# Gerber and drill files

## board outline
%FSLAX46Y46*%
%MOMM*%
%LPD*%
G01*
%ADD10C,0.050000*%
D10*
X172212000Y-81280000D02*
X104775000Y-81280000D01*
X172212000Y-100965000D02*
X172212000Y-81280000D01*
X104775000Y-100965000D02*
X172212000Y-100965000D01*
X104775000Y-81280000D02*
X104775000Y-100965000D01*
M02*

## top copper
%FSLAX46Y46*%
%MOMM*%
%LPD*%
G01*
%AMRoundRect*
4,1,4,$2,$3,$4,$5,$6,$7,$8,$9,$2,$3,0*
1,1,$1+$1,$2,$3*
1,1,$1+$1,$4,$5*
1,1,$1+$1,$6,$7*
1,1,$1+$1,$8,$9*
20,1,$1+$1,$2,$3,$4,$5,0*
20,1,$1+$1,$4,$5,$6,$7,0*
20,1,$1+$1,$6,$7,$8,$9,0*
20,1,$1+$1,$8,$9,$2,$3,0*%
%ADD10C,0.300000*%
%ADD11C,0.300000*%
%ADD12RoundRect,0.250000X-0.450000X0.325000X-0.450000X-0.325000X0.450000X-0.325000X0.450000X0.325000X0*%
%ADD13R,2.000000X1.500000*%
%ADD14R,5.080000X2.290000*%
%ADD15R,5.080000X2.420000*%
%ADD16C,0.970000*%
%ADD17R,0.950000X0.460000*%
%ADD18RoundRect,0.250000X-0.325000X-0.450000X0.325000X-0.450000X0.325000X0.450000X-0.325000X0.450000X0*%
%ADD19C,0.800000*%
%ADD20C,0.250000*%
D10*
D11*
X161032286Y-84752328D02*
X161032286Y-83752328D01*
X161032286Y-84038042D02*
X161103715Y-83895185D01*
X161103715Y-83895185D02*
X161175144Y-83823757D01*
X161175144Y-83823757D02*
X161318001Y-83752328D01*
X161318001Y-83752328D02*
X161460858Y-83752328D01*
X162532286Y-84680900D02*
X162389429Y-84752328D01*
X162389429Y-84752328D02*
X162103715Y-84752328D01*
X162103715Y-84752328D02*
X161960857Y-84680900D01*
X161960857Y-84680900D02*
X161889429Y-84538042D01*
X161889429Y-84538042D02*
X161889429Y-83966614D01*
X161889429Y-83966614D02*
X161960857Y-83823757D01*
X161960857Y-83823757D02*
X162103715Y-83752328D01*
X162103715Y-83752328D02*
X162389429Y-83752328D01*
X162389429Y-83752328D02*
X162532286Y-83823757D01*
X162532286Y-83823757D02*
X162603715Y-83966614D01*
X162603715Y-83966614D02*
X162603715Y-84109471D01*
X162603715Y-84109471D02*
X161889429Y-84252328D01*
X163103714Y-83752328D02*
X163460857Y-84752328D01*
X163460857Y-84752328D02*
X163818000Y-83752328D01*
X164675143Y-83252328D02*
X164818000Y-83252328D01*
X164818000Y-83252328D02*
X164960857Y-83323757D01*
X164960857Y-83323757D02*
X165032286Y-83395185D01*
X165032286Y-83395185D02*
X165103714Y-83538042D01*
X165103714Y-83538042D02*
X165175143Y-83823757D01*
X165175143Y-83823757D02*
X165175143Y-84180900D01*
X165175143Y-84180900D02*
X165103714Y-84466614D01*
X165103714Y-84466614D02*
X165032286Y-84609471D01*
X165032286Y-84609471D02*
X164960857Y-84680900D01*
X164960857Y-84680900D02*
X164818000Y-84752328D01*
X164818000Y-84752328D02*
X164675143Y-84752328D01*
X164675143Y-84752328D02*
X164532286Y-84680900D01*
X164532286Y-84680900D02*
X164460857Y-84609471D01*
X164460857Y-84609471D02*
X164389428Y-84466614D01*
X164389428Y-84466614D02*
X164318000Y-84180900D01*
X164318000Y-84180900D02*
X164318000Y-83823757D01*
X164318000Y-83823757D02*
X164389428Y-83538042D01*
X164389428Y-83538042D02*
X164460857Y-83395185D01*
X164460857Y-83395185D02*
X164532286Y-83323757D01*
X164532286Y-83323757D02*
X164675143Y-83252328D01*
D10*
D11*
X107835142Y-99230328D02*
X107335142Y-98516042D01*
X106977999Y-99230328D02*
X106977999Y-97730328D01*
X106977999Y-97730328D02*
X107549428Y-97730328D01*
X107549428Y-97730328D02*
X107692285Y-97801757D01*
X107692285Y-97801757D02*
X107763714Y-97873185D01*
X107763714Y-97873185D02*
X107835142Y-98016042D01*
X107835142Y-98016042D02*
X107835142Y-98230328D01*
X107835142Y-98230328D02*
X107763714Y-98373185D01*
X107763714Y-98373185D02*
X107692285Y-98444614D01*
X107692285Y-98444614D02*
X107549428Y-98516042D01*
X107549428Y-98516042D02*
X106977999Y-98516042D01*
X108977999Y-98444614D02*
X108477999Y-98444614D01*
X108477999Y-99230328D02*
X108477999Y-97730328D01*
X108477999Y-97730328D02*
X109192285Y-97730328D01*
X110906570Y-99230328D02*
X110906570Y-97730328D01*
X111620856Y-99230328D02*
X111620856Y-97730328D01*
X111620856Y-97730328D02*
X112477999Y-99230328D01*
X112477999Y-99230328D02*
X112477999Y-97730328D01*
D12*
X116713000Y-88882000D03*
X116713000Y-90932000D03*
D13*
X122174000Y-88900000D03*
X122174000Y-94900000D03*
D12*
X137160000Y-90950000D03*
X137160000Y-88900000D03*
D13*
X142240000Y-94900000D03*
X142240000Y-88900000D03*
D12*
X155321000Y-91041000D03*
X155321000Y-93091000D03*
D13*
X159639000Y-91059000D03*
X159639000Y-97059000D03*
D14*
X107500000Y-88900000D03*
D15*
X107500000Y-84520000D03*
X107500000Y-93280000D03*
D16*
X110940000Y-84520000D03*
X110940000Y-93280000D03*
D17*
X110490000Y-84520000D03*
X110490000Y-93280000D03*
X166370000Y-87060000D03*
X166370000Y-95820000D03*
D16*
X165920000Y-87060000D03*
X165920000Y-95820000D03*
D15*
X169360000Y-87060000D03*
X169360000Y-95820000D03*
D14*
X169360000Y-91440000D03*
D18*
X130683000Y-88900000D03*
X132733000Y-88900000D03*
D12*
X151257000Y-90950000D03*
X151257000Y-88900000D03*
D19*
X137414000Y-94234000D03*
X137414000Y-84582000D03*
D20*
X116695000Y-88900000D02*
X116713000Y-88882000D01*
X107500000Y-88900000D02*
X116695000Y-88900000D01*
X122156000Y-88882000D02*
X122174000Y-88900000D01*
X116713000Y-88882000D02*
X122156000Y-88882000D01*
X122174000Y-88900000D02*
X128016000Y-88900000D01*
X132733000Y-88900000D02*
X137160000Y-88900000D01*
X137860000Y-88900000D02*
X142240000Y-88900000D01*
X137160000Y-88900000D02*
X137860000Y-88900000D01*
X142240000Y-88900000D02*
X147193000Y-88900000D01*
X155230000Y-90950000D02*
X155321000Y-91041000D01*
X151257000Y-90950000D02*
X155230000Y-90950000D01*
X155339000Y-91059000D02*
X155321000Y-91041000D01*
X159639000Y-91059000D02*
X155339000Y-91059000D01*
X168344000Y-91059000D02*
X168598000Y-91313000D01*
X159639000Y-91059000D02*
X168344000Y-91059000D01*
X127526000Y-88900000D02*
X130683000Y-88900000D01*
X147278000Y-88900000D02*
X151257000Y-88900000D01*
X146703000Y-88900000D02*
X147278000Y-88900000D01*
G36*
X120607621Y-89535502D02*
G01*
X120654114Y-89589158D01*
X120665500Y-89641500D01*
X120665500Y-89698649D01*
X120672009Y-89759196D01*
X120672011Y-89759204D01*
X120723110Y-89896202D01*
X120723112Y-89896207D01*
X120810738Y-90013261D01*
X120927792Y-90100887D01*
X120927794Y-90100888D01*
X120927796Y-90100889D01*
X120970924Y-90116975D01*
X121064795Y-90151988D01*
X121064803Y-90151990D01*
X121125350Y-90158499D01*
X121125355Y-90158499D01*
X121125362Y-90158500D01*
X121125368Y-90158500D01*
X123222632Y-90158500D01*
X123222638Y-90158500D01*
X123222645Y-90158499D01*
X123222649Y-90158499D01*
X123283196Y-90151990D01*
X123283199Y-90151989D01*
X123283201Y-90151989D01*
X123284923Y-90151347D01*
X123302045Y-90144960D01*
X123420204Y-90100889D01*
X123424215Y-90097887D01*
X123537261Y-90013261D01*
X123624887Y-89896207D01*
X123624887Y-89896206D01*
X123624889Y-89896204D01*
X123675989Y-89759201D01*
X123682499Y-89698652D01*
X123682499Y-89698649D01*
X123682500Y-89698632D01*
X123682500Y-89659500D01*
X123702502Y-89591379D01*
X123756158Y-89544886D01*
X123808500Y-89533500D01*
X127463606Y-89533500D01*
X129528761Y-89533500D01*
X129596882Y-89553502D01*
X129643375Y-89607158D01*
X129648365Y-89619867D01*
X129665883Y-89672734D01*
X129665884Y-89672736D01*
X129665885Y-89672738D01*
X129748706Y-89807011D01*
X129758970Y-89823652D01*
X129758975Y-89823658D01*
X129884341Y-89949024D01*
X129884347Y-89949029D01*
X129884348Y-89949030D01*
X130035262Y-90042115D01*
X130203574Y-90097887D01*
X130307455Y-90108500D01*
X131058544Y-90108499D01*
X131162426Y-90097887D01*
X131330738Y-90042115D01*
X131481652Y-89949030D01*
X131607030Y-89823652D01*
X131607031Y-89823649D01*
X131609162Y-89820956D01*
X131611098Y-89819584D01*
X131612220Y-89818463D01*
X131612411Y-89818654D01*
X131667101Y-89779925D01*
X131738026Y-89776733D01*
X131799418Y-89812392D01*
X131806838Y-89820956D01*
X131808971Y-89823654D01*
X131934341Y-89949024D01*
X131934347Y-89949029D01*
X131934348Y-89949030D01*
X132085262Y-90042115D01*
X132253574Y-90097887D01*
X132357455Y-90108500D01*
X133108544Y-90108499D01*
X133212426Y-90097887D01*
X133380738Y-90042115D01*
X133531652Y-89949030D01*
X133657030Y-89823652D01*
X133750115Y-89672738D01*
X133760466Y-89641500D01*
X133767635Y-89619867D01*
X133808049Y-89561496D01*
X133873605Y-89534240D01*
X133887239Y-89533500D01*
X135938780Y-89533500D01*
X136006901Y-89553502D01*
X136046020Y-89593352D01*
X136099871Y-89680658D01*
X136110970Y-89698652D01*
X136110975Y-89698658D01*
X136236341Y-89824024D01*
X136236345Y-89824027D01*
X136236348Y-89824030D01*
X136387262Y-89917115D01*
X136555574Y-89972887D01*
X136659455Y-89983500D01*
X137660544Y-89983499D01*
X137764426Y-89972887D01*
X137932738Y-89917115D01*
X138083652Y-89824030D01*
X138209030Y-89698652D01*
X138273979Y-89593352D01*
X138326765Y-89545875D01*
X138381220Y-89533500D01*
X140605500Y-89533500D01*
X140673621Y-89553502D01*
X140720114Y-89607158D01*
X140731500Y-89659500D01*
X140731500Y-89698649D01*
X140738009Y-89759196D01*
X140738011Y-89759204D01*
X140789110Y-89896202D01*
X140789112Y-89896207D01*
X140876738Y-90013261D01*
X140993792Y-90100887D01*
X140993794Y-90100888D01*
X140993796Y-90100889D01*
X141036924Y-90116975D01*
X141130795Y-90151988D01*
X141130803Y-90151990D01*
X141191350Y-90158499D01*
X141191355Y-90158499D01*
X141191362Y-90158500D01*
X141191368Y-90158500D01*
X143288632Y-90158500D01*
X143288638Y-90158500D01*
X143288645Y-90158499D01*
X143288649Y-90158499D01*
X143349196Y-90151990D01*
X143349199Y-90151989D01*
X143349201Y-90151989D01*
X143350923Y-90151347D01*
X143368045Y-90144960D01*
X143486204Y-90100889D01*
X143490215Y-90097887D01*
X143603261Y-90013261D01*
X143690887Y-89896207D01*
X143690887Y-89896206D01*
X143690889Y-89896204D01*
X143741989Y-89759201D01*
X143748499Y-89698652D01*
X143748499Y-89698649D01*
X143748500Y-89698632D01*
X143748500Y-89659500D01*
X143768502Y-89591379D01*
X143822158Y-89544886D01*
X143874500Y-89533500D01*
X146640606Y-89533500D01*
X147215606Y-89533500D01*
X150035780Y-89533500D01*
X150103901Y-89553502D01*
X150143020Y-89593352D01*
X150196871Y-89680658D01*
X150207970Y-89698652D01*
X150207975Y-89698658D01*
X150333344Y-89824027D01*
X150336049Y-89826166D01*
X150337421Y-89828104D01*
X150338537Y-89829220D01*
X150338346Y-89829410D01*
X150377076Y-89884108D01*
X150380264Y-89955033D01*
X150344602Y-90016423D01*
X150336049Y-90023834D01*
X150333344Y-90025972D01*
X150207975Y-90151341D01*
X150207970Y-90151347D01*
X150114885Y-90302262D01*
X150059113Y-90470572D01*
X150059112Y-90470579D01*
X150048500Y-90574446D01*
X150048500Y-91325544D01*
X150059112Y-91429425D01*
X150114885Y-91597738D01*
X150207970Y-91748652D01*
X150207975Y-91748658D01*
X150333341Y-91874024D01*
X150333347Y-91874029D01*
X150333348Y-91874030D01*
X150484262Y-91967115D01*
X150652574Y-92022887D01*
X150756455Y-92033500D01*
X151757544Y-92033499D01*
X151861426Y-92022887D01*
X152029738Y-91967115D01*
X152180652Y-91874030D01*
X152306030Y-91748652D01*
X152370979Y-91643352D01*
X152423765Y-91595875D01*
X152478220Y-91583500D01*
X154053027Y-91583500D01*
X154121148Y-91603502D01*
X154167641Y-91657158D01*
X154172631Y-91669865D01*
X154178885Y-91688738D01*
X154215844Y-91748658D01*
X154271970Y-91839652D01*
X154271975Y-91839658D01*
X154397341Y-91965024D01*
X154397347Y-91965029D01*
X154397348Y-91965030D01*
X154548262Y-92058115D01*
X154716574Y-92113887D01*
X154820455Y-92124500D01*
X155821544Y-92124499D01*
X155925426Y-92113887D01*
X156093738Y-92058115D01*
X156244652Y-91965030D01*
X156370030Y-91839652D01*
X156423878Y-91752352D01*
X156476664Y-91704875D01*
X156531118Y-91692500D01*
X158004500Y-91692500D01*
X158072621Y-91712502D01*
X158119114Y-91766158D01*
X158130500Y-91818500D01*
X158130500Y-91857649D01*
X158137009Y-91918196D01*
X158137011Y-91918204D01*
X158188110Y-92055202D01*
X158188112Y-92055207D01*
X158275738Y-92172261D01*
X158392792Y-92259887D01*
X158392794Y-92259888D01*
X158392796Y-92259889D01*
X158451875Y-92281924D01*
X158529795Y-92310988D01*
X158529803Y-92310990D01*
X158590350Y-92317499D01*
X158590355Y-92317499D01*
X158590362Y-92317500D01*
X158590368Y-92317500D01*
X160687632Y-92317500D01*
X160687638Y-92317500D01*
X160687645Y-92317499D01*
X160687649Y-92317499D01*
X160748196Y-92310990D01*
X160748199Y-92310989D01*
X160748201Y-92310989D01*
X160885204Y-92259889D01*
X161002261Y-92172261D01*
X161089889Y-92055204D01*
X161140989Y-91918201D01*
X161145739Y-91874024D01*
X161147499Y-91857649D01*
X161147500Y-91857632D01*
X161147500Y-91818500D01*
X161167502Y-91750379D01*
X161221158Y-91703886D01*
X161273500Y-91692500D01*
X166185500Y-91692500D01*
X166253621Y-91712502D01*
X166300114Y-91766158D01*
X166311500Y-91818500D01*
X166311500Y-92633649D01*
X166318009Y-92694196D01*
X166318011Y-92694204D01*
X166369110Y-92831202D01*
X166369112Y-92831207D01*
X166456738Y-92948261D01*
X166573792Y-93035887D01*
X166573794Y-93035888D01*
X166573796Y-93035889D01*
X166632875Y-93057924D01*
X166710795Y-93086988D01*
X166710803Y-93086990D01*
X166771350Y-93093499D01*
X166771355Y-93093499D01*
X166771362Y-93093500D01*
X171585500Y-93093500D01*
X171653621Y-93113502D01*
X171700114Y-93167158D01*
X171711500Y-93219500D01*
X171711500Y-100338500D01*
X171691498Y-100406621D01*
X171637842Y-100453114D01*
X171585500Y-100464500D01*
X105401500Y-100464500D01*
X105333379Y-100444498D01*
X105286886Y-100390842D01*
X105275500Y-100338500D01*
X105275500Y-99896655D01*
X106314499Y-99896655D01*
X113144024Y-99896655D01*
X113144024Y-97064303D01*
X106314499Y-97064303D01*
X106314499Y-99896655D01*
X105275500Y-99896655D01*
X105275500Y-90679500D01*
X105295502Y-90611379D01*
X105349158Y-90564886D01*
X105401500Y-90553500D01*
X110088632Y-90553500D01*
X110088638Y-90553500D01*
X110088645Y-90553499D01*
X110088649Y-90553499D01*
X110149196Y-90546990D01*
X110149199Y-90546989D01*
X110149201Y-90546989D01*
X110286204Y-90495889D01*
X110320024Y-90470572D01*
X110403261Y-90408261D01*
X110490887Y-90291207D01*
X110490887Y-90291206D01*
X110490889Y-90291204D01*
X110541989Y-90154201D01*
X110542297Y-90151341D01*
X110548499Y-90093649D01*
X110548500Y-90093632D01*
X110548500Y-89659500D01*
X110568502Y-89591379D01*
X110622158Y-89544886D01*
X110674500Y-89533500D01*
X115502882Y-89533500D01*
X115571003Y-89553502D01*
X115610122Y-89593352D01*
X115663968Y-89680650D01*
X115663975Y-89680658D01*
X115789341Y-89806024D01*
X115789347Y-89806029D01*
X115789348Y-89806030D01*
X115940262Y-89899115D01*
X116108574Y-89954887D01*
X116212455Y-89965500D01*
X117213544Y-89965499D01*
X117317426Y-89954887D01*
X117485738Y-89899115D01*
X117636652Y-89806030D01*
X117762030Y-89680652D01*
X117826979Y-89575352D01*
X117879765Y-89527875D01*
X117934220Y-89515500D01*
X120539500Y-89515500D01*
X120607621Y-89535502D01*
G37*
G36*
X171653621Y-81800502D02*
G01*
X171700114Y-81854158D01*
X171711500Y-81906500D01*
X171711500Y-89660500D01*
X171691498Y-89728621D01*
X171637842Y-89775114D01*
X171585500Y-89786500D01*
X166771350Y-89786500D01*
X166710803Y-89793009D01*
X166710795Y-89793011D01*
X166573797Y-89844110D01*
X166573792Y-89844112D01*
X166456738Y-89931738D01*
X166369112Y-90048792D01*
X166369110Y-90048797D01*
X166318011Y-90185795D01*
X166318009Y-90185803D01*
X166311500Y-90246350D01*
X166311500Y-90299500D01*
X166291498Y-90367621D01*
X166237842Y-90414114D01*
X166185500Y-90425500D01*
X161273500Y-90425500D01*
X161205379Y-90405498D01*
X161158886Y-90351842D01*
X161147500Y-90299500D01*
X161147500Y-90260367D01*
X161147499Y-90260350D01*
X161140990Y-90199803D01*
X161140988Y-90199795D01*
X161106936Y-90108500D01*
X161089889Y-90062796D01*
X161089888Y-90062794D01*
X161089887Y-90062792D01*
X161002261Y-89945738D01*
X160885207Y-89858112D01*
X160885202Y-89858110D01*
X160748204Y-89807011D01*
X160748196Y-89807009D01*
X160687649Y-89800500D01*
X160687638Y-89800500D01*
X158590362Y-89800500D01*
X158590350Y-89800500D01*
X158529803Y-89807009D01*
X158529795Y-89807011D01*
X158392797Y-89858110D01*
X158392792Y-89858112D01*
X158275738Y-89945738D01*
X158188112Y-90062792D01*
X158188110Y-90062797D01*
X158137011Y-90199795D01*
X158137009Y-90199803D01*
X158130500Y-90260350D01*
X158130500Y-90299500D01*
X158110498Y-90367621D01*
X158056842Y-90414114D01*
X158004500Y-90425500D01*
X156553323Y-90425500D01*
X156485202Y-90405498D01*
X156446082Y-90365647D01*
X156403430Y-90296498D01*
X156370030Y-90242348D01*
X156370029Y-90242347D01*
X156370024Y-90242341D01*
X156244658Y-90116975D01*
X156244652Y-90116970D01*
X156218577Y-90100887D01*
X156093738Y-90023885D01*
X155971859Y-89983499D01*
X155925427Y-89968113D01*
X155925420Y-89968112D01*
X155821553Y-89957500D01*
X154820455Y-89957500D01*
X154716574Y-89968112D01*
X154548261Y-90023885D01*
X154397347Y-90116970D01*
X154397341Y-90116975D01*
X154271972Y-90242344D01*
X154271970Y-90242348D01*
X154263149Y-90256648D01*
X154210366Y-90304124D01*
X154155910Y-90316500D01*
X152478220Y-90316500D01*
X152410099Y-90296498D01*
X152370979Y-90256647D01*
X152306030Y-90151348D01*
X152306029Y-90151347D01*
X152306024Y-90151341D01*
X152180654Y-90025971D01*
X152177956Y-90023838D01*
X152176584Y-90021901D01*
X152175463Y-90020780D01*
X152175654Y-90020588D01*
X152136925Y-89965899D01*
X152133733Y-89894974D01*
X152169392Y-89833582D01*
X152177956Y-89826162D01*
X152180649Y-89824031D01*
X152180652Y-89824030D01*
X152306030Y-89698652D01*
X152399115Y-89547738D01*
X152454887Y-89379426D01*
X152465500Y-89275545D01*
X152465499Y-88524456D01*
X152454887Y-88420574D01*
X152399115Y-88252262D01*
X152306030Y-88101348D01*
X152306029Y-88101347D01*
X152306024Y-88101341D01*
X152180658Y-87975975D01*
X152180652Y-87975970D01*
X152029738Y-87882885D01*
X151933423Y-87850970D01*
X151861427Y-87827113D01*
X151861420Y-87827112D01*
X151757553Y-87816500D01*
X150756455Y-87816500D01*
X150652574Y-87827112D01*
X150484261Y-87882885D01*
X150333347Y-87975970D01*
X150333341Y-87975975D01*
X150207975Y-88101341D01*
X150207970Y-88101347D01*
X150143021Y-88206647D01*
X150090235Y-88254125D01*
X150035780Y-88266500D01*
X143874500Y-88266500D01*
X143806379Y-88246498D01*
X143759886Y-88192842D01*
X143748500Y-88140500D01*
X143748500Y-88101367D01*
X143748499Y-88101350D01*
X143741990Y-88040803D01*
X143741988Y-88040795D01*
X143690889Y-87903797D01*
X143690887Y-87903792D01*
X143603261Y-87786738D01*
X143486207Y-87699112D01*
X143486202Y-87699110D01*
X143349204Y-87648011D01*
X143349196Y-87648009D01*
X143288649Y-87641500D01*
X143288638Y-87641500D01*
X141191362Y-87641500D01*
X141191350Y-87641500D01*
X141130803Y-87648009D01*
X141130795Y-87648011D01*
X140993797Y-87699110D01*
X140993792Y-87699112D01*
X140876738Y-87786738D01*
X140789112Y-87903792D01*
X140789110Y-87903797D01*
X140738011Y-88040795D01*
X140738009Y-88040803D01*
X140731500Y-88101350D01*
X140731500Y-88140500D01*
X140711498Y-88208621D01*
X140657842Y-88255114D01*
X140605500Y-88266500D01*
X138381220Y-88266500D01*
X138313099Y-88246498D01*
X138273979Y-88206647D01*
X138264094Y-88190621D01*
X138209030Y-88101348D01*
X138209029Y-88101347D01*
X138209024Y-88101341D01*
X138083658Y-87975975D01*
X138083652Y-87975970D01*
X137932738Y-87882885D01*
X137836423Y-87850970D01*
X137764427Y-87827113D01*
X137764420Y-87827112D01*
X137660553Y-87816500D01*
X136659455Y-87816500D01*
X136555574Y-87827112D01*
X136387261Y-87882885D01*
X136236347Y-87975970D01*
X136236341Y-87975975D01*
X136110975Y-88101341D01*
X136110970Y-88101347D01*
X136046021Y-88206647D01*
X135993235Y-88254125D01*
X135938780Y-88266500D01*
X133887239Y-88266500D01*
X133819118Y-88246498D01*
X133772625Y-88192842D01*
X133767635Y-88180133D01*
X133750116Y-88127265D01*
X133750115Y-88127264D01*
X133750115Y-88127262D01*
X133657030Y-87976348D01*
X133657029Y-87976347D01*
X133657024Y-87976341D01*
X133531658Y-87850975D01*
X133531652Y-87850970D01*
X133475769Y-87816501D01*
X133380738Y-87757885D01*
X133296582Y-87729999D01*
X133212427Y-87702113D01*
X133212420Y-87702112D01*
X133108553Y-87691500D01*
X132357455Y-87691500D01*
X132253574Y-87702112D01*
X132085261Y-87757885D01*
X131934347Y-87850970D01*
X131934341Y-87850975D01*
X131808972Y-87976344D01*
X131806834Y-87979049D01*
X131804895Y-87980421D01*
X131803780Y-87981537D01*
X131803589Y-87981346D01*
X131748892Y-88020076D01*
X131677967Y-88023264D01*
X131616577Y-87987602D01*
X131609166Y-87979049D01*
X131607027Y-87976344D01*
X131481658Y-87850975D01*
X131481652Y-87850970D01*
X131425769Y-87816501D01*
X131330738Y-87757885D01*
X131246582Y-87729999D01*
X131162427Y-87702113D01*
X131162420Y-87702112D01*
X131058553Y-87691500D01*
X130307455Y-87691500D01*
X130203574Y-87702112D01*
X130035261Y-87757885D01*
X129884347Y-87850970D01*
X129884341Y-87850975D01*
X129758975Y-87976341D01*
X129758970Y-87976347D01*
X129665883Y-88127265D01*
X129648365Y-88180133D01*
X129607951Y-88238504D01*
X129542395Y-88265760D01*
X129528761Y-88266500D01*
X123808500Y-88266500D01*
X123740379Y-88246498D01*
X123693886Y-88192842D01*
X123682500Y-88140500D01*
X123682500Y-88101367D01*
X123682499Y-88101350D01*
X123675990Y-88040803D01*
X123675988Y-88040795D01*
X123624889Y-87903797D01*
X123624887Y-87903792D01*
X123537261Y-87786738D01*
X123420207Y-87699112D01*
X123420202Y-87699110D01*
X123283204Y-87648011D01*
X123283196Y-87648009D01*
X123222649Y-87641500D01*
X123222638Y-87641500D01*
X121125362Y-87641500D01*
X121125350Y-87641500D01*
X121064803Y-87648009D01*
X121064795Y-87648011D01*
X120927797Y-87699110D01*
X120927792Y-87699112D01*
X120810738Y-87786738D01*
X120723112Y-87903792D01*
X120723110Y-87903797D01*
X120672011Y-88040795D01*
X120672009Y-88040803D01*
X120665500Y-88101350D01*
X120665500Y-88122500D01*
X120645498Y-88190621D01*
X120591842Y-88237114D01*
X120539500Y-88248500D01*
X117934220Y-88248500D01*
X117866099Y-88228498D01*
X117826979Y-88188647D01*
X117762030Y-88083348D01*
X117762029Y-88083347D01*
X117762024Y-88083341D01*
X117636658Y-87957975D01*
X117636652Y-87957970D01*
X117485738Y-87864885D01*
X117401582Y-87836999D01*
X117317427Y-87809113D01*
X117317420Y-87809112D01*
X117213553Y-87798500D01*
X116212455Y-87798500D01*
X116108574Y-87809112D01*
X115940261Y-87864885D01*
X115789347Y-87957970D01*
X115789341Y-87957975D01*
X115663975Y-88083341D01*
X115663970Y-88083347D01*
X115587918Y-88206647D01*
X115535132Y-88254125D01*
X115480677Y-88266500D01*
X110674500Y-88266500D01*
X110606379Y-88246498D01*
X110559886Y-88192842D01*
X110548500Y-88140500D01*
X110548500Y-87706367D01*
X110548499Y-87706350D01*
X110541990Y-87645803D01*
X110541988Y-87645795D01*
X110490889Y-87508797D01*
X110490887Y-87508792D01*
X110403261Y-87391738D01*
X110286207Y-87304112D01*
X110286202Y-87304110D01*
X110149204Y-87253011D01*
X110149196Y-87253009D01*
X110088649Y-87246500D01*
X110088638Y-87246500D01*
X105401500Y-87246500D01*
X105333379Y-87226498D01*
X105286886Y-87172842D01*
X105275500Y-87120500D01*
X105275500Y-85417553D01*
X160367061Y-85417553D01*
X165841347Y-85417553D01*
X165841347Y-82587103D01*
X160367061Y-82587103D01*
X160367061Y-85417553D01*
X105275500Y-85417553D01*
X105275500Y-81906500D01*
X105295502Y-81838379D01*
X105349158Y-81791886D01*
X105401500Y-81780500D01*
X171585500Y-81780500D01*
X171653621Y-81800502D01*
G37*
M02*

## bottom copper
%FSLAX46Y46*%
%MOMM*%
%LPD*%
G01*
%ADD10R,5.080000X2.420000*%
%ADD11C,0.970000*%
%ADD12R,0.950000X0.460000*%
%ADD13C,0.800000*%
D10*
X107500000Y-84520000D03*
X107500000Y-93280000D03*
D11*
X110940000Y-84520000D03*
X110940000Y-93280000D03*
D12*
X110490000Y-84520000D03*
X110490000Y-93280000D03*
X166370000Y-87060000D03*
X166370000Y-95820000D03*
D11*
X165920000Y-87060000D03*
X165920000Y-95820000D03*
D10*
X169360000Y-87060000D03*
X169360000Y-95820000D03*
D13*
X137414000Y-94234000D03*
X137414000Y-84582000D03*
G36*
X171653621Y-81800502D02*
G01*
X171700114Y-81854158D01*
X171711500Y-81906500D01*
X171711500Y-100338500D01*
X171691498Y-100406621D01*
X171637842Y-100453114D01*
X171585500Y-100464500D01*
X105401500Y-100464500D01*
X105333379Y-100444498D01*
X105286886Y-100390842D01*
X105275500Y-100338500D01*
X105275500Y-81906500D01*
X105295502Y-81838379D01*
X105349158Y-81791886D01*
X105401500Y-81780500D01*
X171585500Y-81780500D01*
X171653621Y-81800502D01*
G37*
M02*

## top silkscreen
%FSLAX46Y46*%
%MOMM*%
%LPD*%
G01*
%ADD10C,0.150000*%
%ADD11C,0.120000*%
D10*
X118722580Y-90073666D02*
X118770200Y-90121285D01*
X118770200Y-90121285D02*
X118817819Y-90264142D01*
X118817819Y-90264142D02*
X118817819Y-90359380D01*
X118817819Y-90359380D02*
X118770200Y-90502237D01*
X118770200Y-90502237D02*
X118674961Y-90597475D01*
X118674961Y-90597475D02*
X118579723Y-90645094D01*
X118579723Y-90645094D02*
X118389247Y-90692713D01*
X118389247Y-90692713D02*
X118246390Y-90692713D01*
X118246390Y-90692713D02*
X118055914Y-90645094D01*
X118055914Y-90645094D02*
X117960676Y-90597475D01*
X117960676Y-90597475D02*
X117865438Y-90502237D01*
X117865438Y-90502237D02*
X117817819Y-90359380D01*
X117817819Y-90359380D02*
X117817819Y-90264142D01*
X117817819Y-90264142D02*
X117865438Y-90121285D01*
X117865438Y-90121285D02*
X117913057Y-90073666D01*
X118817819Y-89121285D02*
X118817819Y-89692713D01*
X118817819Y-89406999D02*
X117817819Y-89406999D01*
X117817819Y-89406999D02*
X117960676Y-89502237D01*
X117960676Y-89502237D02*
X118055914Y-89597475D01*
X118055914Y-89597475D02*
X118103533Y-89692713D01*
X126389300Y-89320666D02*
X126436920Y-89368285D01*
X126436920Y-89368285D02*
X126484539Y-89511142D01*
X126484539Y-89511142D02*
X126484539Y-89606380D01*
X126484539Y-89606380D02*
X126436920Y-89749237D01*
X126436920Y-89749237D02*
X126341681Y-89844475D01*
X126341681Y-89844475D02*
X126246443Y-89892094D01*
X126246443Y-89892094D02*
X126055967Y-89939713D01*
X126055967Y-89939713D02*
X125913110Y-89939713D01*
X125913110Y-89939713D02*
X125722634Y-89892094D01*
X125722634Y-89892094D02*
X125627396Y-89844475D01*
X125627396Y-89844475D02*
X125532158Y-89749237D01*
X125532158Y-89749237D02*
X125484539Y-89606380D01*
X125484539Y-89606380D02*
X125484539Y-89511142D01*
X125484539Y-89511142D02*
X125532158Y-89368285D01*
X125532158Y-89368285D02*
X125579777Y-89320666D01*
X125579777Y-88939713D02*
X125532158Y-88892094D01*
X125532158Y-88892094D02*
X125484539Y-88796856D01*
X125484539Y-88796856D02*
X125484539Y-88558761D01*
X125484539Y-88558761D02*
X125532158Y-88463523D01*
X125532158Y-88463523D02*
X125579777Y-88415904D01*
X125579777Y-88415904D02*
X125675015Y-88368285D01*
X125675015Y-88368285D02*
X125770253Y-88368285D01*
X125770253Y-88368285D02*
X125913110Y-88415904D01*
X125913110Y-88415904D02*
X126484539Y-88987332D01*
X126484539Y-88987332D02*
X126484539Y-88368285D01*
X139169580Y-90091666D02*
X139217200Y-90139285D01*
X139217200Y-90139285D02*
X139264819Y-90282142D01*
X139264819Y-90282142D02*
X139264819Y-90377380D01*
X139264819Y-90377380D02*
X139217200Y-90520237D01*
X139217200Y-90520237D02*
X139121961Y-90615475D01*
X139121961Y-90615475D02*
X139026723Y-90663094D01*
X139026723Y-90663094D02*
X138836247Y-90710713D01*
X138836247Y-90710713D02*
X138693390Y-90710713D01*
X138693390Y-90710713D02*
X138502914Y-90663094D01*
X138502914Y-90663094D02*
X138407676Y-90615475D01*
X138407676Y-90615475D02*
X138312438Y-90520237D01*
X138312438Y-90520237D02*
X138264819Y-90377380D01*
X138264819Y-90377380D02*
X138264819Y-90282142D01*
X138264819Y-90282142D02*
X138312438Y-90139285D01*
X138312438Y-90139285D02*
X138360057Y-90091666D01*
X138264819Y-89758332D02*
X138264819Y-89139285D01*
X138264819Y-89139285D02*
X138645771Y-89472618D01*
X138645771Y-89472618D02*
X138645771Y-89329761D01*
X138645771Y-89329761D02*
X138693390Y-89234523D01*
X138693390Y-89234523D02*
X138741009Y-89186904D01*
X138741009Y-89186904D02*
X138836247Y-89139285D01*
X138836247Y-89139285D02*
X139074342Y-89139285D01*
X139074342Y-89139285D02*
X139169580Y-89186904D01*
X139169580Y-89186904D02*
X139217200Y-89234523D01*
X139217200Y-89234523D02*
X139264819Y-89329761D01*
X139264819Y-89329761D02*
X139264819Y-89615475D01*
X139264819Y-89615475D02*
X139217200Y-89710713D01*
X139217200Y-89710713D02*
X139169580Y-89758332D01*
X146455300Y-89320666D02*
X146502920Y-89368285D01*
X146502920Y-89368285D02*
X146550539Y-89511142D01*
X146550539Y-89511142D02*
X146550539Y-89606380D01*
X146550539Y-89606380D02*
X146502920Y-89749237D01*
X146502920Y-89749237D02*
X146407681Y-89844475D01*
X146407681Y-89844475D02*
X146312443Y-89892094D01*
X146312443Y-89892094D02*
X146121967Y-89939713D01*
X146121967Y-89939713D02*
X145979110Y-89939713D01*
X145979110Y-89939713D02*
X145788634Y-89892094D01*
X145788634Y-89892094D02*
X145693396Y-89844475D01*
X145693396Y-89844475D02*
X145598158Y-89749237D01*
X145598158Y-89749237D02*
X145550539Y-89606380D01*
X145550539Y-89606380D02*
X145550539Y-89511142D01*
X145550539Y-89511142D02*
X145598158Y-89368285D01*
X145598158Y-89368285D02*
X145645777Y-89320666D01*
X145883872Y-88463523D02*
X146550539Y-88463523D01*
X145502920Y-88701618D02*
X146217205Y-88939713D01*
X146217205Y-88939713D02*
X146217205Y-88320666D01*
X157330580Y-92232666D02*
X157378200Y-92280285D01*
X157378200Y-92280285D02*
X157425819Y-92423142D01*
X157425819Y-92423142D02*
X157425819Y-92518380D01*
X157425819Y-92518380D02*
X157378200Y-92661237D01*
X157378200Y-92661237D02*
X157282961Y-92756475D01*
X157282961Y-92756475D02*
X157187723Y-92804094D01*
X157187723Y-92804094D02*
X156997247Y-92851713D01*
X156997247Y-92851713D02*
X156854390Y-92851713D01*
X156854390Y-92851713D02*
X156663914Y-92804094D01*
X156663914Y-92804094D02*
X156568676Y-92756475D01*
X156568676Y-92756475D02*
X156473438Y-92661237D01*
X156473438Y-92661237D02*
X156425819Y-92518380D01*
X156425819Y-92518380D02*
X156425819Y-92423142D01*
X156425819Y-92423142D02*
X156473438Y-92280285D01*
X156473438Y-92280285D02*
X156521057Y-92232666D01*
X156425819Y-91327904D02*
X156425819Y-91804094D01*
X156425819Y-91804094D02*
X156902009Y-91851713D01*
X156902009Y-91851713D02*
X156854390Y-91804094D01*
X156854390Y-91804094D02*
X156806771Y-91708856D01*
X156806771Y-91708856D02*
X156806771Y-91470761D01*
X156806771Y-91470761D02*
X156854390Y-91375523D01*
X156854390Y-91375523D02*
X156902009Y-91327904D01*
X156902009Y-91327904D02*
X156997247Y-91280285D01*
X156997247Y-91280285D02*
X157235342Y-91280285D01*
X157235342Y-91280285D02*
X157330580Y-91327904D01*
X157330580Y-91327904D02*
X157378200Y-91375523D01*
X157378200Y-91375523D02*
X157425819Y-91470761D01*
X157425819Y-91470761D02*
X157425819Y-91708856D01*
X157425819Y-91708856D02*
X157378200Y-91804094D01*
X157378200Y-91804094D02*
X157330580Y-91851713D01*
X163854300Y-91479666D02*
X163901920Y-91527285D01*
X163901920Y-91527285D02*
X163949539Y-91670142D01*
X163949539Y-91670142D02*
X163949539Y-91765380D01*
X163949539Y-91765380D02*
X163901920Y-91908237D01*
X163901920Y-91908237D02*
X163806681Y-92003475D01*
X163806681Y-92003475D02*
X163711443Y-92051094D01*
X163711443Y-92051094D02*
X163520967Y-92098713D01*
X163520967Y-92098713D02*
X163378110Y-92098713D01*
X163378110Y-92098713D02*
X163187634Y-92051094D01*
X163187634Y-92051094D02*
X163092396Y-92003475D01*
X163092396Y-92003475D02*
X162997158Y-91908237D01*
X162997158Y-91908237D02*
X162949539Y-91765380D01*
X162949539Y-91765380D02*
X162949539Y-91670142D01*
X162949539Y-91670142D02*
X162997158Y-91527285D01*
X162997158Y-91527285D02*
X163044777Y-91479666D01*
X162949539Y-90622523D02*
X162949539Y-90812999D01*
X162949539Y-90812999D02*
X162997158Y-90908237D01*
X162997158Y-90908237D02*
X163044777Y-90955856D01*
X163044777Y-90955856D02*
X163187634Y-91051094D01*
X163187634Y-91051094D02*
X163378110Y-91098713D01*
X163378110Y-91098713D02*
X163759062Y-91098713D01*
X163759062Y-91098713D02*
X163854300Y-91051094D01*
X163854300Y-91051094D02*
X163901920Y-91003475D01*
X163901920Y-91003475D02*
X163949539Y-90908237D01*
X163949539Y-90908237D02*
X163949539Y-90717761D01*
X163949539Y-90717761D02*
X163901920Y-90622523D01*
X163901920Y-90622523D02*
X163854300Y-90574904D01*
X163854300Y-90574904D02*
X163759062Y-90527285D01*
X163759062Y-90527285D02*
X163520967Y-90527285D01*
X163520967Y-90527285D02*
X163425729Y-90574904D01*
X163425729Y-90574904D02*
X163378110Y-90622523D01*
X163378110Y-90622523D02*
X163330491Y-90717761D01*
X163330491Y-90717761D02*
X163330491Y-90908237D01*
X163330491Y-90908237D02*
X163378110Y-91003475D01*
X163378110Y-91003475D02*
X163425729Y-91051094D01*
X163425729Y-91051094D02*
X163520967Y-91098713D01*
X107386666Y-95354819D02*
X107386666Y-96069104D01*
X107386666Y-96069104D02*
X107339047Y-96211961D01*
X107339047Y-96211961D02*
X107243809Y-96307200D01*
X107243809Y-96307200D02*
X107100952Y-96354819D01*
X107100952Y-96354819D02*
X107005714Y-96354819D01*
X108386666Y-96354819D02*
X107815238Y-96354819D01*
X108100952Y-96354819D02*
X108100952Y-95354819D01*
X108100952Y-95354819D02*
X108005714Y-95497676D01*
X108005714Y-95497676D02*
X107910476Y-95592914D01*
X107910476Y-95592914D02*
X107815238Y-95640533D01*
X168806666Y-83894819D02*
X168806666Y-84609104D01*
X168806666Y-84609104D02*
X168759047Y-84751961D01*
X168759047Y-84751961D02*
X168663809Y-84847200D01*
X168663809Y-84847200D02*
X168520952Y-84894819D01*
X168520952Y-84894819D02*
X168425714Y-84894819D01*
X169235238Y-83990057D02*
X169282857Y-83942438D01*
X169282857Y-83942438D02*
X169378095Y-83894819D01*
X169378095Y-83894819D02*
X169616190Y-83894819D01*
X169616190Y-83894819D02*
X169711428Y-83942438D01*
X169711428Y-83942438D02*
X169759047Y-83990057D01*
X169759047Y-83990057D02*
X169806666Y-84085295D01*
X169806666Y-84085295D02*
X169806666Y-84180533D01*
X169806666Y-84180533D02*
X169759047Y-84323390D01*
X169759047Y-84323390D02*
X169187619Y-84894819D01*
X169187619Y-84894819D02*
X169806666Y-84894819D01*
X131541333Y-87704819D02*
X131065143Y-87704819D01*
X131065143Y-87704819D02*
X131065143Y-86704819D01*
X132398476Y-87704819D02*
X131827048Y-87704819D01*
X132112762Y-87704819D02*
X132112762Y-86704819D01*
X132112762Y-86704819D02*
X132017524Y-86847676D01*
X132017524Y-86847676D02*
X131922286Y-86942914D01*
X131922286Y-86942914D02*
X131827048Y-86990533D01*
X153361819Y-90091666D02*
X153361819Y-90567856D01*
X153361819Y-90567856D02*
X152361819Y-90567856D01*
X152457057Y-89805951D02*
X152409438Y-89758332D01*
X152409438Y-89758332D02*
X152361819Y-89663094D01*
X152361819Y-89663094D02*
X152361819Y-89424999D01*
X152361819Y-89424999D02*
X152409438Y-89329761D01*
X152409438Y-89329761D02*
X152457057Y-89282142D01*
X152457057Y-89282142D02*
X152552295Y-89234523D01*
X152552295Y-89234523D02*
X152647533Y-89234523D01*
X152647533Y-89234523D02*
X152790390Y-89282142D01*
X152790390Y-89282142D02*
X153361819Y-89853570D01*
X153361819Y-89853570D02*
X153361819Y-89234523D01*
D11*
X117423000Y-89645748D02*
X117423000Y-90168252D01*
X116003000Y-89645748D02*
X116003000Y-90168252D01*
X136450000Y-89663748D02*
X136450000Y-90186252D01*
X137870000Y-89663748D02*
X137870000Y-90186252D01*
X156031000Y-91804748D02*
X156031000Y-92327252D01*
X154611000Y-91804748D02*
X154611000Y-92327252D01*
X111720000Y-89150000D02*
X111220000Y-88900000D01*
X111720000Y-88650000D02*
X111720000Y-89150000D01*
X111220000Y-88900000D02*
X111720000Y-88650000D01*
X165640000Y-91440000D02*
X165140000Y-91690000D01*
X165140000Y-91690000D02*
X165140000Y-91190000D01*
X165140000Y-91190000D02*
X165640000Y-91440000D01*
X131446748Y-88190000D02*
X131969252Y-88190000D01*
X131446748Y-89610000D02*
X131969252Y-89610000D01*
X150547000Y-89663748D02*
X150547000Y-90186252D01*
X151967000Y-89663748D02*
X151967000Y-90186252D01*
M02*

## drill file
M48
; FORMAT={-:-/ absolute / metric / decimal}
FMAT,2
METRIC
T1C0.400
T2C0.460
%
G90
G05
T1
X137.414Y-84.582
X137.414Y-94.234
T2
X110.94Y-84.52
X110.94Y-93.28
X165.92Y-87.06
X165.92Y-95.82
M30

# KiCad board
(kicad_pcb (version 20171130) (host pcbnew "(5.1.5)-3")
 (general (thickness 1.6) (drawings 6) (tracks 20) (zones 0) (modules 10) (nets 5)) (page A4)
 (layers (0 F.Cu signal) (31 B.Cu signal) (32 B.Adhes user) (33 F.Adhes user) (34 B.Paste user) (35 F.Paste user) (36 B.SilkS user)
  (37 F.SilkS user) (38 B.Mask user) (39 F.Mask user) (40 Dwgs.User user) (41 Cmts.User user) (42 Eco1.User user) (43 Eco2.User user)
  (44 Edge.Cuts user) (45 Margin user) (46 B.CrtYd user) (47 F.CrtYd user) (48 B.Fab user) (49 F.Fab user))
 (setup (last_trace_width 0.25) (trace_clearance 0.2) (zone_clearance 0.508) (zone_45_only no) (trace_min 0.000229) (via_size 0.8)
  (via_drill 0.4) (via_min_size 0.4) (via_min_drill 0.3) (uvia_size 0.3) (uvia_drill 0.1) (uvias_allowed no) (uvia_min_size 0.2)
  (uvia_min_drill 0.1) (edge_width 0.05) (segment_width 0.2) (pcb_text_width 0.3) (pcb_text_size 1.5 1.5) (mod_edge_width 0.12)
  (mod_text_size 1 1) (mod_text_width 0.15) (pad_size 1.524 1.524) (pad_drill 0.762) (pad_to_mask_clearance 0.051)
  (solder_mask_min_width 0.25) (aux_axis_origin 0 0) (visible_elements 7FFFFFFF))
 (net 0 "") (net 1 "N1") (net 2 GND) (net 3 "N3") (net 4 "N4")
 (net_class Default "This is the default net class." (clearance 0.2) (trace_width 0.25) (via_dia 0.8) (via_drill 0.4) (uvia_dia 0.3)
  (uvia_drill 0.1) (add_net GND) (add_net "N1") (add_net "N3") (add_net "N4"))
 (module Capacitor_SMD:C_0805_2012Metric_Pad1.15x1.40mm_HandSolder (layer F.Cu) (at 116.713 89.907 270)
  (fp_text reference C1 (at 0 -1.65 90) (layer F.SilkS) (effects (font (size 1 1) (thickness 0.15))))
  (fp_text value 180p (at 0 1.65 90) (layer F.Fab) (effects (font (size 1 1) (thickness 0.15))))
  (fp_line (start -0.261252 -0.71) (end 0.261252 -0.71) (layer F.SilkS) (width 0.12))
  (fp_line (start -0.261252 0.71) (end 0.261252 0.71) (layer F.SilkS) (width 0.12))
  (pad 1 smd roundrect (at -1.025 0 270) (size 1.15 1.4) (layers F.Cu F.Paste F.Mask) (roundrect_rratio 0.217391) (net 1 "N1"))
  (pad 2 smd roundrect (at 1.025 0 270) (size 1.15 1.4) (layers F.Cu F.Paste F.Mask) (roundrect_rratio 0.217391) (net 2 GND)))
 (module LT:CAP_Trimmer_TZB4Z (layer F.Cu) (at 122.174 88.9 270)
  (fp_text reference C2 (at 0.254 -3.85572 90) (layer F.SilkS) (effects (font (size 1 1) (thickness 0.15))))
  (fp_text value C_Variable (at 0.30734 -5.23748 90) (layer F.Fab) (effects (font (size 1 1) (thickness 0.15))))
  (pad 1 smd rect (at 0 0 270) (size 1.5 2) (layers F.Cu F.Paste F.Mask) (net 1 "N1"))
  (pad 2 smd rect (at 6 0 270) (size 1.5 2) (layers F.Cu F.Paste F.Mask) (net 2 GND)))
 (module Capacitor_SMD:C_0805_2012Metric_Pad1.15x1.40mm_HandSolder (layer F.Cu) (at 137.16 89.925 270)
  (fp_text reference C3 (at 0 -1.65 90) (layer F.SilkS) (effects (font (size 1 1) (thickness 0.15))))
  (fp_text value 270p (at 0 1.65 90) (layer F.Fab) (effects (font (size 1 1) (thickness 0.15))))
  (fp_line (start -0.261252 0.71) (end 0.261252 0.71) (layer F.SilkS) (width 0.12))
  (fp_line (start -0.261252 -0.71) (end 0.261252 -0.71) (layer F.SilkS) (width 0.12))
  (pad 2 smd roundrect (at 1.025 0 270) (size 1.15 1.4) (layers F.Cu F.Paste F.Mask) (roundrect_rratio 0.217391) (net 2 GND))
  (pad 1 smd roundrect (at -1.025 0 270) (size 1.15 1.4) (layers F.Cu F.Paste F.Mask) (roundrect_rratio 0.217391) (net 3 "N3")))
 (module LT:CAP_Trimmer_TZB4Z (layer F.Cu) (at 142.24 88.9 270)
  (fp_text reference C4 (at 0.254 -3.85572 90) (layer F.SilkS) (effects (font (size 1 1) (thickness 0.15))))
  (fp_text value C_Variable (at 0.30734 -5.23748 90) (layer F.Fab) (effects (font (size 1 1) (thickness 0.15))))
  (pad 2 smd rect (at 6 0 270) (size 1.5 2) (layers F.Cu F.Paste F.Mask) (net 2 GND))
  (pad 1 smd rect (at 0 0 270) (size 1.5 2) (layers F.Cu F.Paste F.Mask) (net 3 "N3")))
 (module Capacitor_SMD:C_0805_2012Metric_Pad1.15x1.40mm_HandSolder (layer F.Cu) (at 155.321 92.066 270)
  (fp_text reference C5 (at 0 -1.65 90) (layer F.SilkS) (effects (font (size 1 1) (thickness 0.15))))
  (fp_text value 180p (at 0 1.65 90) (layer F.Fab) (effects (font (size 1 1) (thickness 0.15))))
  (fp_line (start -0.261252 -0.71) (end 0.261252 -0.71) (layer F.SilkS) (width 0.12))
  (fp_line (start -0.261252 0.71) (end 0.261252 0.71) (layer F.SilkS) (width 0.12))
  (pad 1 smd roundrect (at -1.025 0 270) (size 1.15 1.4) (layers F.Cu F.Paste F.Mask) (roundrect_rratio 0.217391) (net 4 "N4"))
  (pad 2 smd roundrect (at 1.025 0 270) (size 1.15 1.4) (layers F.Cu F.Paste F.Mask) (roundrect_rratio 0.217391) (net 2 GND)))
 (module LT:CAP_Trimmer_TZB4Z (layer F.Cu) (at 159.639 91.059 270)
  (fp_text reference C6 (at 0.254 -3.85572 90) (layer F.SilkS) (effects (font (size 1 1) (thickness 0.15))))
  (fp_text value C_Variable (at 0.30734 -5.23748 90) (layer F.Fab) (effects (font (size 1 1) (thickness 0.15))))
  (pad 1 smd rect (at 0 0 270) (size 1.5 2) (layers F.Cu F.Paste F.Mask) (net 4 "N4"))
  (pad 2 smd rect (at 6 0 270) (size 1.5 2) (layers F.Cu F.Paste F.Mask) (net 2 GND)))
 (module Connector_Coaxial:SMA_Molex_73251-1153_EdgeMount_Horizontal (layer F.Cu) (at 109.22 88.9)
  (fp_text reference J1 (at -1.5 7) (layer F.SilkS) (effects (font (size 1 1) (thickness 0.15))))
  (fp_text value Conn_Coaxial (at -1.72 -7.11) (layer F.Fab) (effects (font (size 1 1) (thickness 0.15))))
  (fp_line (start 2.5 0.25) (end 2 0) (layer F.SilkS) (width 0.12))
  (fp_line (start 2.5 -0.25) (end 2.5 0.25) (layer F.SilkS) (width 0.12))
  (fp_line (start 2 0) (end 2.5 -0.25) (layer F.SilkS) (width 0.12))
  (pad 1 smd rect (at -1.72 0) (size 5.08 2.29) (layers F.Cu F.Paste F.Mask) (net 1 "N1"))
  (pad 2 smd rect (at -1.72 -4.38) (size 5.08 2.42) (layers F.Cu F.Paste F.Mask) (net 2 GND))
  (pad 2 smd rect (at -1.72 4.38) (size 5.08 2.42) (layers F.Cu F.Paste F.Mask) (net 2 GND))
  (pad 2 smd rect (at -1.72 -4.38) (size 5.08 2.42) (layers B.Cu B.Paste B.Mask) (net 2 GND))
  (pad 2 smd rect (at -1.72 4.38) (size 5.08 2.42) (layers B.Cu B.Paste B.Mask) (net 2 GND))
  (pad 2 thru_hole circle (at 1.72 -4.38) (size 0.97 0.97) (drill 0.46) (layers *.Cu) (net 2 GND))
  (pad 2 thru_hole circle (at 1.72 4.38) (size 0.97 0.97) (drill 0.46) (layers *.Cu) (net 2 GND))
  (pad 2 smd rect (at 1.27 -4.38) (size 0.95 0.46) (layers F.Cu) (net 2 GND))
  (pad 2 smd rect (at 1.27 4.38) (size 0.95 0.46) (layers F.Cu) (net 2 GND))
  (pad 2 smd rect (at 1.27 -4.38) (size 0.95 0.46) (layers B.Cu) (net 2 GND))
  (pad 2 smd rect (at 1.27 4.38) (size 0.95 0.46) (layers B.Cu) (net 2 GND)))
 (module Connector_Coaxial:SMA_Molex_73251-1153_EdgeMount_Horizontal (layer F.Cu) (at 167.64 91.44 180)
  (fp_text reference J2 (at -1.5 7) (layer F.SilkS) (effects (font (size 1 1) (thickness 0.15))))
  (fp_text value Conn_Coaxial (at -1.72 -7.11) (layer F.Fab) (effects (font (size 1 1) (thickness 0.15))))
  (fp_line (start 2 0) (end 2.5 -0.25) (layer F.SilkS) (width 0.12))
  (fp_line (start 2.5 -0.25) (end 2.5 0.25) (layer F.SilkS) (width 0.12))
  (fp_line (start 2.5 0.25) (end 2 0) (layer F.SilkS) (width 0.12))
  (pad 2 smd rect (at 1.27 4.38 180) (size 0.95 0.46) (layers B.Cu) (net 2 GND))
  (pad 2 smd rect (at 1.27 -4.38 180) (size 0.95 0.46) (layers B.Cu) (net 2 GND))
  (pad 2 smd rect (at 1.27 4.38 180) (size 0.95 0.46) (layers F.Cu) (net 2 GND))
  (pad 2 smd rect (at 1.27 -4.38 180) (size 0.95 0.46) (layers F.Cu) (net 2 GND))
  (pad 2 thru_hole circle (at 1.72 4.38 180) (size 0.97 0.97) (drill 0.46) (layers *.Cu) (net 2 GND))
  (pad 2 thru_hole circle (at 1.72 -4.38 180) (size 0.97 0.97) (drill 0.46) (layers *.Cu) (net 2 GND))
  (pad 2 smd rect (at -1.72 4.38 180) (size 5.08 2.42) (layers B.Cu B.Paste B.Mask) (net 2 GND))
  (pad 2 smd rect (at -1.72 -4.38 180) (size 5.08 2.42) (layers B.Cu B.Paste B.Mask) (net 2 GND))
  (pad 2 smd rect (at -1.72 4.38 180) (size 5.08 2.42) (layers F.Cu F.Paste F.Mask) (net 2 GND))
  (pad 2 smd rect (at -1.72 -4.38 180) (size 5.08 2.42) (layers F.Cu F.Paste F.Mask) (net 2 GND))
  (pad 1 smd rect (at -1.72 0 180) (size 5.08 2.29) (layers F.Cu F.Paste F.Mask) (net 4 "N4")))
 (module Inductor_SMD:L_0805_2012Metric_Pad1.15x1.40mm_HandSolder (layer F.Cu) (at 131.708 88.9)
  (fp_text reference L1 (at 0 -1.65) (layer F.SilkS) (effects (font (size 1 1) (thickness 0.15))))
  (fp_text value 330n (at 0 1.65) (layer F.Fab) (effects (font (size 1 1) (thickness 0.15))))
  (fp_line (start -0.261252 -0.71) (end 0.261252 -0.71) (layer F.SilkS) (width 0.12))
  (fp_line (start -0.261252 0.71) (end 0.261252 0.71) (layer F.SilkS) (width 0.12))
  (pad 1 smd roundrect (at -1.025 0) (size 1.15 1.4) (layers F.Cu F.Paste F.Mask) (roundrect_rratio 0.217391) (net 1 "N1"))
  (pad 2 smd roundrect (at 1.025 0) (size 1.15 1.4) (layers F.Cu F.Paste F.Mask) (roundrect_rratio 0.217391) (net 3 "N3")))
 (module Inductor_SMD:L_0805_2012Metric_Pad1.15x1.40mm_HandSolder (layer F.Cu) (at 151.257 89.925 270)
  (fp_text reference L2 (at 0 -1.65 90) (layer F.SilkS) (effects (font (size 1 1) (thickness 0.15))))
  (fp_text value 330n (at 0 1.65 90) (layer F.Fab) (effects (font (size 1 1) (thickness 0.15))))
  (fp_line (start -0.261252 0.71) (end 0.261252 0.71) (layer F.SilkS) (width 0.12))
  (fp_line (start -0.261252 -0.71) (end 0.261252 -0.71) (layer F.SilkS) (width 0.12))
  (pad 2 smd roundrect (at 1.025 0 270) (size 1.15 1.4) (layers F.Cu F.Paste F.Mask) (roundrect_rratio 0.217391) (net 4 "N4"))
  (pad 1 smd roundrect (at -1.025 0 270) (size 1.15 1.4) (layers F.Cu F.Paste F.Mask) (roundrect_rratio 0.217391) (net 3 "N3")))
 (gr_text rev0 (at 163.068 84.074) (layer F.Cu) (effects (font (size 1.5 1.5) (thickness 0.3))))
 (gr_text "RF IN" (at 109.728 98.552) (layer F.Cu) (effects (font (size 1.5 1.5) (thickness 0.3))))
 (gr_line (start 172.212 81.28) (end 104.775 81.28) (layer Edge.Cuts) (width 0.05))
 (gr_line (start 172.212 100.965) (end 172.212 81.28) (layer Edge.Cuts) (width 0.05))
 (gr_line (start 104.775 100.965) (end 172.212 100.965) (layer Edge.Cuts) (width 0.05))
 (gr_line (start 104.775 81.28) (end 104.775 100.965) (layer Edge.Cuts) (width 0.05))
 (segment (start 116.695 88.9) (end 116.713 88.882) (width 0.25) (layer F.Cu) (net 1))
 (segment (start 107.5 88.9) (end 116.695 88.9) (width 0.25) (layer F.Cu) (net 1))
 (segment (start 122.156 88.882) (end 122.174 88.9) (width 0.25) (layer F.Cu) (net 1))
 (segment (start 116.713 88.882) (end 122.156 88.882) (width 0.25) (layer F.Cu) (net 1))
 (segment (start 122.174 88.9) (end 128.016 88.9) (width 0.25) (layer F.Cu) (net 1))
 (via (at 137.414 94.234) (size 0.8) (drill 0.4) (layers F.Cu B.Cu) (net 2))
 (via (at 137.414 84.582) (size 0.8) (drill 0.4) (layers F.Cu B.Cu) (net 2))
 (segment (start 132.733 88.9) (end 137.16 88.9) (width 0.25) (layer F.Cu) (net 3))
 (segment (start 137.86 88.9) (end 142.24 88.9) (width 0.25) (layer F.Cu) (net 3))
 (segment (start 137.16 88.9) (end 137.86 88.9) (width 0.25) (layer F.Cu) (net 3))
 (segment (start 142.24 88.9) (end 147.193 88.9) (width 0.25) (layer F.Cu) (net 3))
 (segment (start 155.23 90.95) (end 155.321 91.041) (width 0.25) (layer F.Cu) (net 4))
 (segment (start 151.257 90.95) (end 155.23 90.95) (width 0.25) (layer F.Cu) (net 4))
 (segment (start 155.339 91.059) (end 155.321 91.041) (width 0.25) (layer F.Cu) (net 4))
 (segment (start 159.639 91.059) (end 155.339 91.059) (width 0.25) (layer F.Cu) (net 4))
 (segment (start 168.344 91.059) (end 168.598 91.313) (width 0.25) (layer F.Cu) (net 4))
 (segment (start 159.639 91.059) (end 168.344 91.059) (width 0.25) (layer F.Cu) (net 4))
 (segment (start 127.526 88.9) (end 130.683 88.9) (width 0.25) (layer F.Cu) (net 1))
 (segment (start 147.278 88.9) (end 151.257 88.9) (width 0.25) (layer F.Cu) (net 3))
 (segment (start 146.703 88.9) (end 147.278 88.9) (width 0.25) (layer F.Cu) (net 3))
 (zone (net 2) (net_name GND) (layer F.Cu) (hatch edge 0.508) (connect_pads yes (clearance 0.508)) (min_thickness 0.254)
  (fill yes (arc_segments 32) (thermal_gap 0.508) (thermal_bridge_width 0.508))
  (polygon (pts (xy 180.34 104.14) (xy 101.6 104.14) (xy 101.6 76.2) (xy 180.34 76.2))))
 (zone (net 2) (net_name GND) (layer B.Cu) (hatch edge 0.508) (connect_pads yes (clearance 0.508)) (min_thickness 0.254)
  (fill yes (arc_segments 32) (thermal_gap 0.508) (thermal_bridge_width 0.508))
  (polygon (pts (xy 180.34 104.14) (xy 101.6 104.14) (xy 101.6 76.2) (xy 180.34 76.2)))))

